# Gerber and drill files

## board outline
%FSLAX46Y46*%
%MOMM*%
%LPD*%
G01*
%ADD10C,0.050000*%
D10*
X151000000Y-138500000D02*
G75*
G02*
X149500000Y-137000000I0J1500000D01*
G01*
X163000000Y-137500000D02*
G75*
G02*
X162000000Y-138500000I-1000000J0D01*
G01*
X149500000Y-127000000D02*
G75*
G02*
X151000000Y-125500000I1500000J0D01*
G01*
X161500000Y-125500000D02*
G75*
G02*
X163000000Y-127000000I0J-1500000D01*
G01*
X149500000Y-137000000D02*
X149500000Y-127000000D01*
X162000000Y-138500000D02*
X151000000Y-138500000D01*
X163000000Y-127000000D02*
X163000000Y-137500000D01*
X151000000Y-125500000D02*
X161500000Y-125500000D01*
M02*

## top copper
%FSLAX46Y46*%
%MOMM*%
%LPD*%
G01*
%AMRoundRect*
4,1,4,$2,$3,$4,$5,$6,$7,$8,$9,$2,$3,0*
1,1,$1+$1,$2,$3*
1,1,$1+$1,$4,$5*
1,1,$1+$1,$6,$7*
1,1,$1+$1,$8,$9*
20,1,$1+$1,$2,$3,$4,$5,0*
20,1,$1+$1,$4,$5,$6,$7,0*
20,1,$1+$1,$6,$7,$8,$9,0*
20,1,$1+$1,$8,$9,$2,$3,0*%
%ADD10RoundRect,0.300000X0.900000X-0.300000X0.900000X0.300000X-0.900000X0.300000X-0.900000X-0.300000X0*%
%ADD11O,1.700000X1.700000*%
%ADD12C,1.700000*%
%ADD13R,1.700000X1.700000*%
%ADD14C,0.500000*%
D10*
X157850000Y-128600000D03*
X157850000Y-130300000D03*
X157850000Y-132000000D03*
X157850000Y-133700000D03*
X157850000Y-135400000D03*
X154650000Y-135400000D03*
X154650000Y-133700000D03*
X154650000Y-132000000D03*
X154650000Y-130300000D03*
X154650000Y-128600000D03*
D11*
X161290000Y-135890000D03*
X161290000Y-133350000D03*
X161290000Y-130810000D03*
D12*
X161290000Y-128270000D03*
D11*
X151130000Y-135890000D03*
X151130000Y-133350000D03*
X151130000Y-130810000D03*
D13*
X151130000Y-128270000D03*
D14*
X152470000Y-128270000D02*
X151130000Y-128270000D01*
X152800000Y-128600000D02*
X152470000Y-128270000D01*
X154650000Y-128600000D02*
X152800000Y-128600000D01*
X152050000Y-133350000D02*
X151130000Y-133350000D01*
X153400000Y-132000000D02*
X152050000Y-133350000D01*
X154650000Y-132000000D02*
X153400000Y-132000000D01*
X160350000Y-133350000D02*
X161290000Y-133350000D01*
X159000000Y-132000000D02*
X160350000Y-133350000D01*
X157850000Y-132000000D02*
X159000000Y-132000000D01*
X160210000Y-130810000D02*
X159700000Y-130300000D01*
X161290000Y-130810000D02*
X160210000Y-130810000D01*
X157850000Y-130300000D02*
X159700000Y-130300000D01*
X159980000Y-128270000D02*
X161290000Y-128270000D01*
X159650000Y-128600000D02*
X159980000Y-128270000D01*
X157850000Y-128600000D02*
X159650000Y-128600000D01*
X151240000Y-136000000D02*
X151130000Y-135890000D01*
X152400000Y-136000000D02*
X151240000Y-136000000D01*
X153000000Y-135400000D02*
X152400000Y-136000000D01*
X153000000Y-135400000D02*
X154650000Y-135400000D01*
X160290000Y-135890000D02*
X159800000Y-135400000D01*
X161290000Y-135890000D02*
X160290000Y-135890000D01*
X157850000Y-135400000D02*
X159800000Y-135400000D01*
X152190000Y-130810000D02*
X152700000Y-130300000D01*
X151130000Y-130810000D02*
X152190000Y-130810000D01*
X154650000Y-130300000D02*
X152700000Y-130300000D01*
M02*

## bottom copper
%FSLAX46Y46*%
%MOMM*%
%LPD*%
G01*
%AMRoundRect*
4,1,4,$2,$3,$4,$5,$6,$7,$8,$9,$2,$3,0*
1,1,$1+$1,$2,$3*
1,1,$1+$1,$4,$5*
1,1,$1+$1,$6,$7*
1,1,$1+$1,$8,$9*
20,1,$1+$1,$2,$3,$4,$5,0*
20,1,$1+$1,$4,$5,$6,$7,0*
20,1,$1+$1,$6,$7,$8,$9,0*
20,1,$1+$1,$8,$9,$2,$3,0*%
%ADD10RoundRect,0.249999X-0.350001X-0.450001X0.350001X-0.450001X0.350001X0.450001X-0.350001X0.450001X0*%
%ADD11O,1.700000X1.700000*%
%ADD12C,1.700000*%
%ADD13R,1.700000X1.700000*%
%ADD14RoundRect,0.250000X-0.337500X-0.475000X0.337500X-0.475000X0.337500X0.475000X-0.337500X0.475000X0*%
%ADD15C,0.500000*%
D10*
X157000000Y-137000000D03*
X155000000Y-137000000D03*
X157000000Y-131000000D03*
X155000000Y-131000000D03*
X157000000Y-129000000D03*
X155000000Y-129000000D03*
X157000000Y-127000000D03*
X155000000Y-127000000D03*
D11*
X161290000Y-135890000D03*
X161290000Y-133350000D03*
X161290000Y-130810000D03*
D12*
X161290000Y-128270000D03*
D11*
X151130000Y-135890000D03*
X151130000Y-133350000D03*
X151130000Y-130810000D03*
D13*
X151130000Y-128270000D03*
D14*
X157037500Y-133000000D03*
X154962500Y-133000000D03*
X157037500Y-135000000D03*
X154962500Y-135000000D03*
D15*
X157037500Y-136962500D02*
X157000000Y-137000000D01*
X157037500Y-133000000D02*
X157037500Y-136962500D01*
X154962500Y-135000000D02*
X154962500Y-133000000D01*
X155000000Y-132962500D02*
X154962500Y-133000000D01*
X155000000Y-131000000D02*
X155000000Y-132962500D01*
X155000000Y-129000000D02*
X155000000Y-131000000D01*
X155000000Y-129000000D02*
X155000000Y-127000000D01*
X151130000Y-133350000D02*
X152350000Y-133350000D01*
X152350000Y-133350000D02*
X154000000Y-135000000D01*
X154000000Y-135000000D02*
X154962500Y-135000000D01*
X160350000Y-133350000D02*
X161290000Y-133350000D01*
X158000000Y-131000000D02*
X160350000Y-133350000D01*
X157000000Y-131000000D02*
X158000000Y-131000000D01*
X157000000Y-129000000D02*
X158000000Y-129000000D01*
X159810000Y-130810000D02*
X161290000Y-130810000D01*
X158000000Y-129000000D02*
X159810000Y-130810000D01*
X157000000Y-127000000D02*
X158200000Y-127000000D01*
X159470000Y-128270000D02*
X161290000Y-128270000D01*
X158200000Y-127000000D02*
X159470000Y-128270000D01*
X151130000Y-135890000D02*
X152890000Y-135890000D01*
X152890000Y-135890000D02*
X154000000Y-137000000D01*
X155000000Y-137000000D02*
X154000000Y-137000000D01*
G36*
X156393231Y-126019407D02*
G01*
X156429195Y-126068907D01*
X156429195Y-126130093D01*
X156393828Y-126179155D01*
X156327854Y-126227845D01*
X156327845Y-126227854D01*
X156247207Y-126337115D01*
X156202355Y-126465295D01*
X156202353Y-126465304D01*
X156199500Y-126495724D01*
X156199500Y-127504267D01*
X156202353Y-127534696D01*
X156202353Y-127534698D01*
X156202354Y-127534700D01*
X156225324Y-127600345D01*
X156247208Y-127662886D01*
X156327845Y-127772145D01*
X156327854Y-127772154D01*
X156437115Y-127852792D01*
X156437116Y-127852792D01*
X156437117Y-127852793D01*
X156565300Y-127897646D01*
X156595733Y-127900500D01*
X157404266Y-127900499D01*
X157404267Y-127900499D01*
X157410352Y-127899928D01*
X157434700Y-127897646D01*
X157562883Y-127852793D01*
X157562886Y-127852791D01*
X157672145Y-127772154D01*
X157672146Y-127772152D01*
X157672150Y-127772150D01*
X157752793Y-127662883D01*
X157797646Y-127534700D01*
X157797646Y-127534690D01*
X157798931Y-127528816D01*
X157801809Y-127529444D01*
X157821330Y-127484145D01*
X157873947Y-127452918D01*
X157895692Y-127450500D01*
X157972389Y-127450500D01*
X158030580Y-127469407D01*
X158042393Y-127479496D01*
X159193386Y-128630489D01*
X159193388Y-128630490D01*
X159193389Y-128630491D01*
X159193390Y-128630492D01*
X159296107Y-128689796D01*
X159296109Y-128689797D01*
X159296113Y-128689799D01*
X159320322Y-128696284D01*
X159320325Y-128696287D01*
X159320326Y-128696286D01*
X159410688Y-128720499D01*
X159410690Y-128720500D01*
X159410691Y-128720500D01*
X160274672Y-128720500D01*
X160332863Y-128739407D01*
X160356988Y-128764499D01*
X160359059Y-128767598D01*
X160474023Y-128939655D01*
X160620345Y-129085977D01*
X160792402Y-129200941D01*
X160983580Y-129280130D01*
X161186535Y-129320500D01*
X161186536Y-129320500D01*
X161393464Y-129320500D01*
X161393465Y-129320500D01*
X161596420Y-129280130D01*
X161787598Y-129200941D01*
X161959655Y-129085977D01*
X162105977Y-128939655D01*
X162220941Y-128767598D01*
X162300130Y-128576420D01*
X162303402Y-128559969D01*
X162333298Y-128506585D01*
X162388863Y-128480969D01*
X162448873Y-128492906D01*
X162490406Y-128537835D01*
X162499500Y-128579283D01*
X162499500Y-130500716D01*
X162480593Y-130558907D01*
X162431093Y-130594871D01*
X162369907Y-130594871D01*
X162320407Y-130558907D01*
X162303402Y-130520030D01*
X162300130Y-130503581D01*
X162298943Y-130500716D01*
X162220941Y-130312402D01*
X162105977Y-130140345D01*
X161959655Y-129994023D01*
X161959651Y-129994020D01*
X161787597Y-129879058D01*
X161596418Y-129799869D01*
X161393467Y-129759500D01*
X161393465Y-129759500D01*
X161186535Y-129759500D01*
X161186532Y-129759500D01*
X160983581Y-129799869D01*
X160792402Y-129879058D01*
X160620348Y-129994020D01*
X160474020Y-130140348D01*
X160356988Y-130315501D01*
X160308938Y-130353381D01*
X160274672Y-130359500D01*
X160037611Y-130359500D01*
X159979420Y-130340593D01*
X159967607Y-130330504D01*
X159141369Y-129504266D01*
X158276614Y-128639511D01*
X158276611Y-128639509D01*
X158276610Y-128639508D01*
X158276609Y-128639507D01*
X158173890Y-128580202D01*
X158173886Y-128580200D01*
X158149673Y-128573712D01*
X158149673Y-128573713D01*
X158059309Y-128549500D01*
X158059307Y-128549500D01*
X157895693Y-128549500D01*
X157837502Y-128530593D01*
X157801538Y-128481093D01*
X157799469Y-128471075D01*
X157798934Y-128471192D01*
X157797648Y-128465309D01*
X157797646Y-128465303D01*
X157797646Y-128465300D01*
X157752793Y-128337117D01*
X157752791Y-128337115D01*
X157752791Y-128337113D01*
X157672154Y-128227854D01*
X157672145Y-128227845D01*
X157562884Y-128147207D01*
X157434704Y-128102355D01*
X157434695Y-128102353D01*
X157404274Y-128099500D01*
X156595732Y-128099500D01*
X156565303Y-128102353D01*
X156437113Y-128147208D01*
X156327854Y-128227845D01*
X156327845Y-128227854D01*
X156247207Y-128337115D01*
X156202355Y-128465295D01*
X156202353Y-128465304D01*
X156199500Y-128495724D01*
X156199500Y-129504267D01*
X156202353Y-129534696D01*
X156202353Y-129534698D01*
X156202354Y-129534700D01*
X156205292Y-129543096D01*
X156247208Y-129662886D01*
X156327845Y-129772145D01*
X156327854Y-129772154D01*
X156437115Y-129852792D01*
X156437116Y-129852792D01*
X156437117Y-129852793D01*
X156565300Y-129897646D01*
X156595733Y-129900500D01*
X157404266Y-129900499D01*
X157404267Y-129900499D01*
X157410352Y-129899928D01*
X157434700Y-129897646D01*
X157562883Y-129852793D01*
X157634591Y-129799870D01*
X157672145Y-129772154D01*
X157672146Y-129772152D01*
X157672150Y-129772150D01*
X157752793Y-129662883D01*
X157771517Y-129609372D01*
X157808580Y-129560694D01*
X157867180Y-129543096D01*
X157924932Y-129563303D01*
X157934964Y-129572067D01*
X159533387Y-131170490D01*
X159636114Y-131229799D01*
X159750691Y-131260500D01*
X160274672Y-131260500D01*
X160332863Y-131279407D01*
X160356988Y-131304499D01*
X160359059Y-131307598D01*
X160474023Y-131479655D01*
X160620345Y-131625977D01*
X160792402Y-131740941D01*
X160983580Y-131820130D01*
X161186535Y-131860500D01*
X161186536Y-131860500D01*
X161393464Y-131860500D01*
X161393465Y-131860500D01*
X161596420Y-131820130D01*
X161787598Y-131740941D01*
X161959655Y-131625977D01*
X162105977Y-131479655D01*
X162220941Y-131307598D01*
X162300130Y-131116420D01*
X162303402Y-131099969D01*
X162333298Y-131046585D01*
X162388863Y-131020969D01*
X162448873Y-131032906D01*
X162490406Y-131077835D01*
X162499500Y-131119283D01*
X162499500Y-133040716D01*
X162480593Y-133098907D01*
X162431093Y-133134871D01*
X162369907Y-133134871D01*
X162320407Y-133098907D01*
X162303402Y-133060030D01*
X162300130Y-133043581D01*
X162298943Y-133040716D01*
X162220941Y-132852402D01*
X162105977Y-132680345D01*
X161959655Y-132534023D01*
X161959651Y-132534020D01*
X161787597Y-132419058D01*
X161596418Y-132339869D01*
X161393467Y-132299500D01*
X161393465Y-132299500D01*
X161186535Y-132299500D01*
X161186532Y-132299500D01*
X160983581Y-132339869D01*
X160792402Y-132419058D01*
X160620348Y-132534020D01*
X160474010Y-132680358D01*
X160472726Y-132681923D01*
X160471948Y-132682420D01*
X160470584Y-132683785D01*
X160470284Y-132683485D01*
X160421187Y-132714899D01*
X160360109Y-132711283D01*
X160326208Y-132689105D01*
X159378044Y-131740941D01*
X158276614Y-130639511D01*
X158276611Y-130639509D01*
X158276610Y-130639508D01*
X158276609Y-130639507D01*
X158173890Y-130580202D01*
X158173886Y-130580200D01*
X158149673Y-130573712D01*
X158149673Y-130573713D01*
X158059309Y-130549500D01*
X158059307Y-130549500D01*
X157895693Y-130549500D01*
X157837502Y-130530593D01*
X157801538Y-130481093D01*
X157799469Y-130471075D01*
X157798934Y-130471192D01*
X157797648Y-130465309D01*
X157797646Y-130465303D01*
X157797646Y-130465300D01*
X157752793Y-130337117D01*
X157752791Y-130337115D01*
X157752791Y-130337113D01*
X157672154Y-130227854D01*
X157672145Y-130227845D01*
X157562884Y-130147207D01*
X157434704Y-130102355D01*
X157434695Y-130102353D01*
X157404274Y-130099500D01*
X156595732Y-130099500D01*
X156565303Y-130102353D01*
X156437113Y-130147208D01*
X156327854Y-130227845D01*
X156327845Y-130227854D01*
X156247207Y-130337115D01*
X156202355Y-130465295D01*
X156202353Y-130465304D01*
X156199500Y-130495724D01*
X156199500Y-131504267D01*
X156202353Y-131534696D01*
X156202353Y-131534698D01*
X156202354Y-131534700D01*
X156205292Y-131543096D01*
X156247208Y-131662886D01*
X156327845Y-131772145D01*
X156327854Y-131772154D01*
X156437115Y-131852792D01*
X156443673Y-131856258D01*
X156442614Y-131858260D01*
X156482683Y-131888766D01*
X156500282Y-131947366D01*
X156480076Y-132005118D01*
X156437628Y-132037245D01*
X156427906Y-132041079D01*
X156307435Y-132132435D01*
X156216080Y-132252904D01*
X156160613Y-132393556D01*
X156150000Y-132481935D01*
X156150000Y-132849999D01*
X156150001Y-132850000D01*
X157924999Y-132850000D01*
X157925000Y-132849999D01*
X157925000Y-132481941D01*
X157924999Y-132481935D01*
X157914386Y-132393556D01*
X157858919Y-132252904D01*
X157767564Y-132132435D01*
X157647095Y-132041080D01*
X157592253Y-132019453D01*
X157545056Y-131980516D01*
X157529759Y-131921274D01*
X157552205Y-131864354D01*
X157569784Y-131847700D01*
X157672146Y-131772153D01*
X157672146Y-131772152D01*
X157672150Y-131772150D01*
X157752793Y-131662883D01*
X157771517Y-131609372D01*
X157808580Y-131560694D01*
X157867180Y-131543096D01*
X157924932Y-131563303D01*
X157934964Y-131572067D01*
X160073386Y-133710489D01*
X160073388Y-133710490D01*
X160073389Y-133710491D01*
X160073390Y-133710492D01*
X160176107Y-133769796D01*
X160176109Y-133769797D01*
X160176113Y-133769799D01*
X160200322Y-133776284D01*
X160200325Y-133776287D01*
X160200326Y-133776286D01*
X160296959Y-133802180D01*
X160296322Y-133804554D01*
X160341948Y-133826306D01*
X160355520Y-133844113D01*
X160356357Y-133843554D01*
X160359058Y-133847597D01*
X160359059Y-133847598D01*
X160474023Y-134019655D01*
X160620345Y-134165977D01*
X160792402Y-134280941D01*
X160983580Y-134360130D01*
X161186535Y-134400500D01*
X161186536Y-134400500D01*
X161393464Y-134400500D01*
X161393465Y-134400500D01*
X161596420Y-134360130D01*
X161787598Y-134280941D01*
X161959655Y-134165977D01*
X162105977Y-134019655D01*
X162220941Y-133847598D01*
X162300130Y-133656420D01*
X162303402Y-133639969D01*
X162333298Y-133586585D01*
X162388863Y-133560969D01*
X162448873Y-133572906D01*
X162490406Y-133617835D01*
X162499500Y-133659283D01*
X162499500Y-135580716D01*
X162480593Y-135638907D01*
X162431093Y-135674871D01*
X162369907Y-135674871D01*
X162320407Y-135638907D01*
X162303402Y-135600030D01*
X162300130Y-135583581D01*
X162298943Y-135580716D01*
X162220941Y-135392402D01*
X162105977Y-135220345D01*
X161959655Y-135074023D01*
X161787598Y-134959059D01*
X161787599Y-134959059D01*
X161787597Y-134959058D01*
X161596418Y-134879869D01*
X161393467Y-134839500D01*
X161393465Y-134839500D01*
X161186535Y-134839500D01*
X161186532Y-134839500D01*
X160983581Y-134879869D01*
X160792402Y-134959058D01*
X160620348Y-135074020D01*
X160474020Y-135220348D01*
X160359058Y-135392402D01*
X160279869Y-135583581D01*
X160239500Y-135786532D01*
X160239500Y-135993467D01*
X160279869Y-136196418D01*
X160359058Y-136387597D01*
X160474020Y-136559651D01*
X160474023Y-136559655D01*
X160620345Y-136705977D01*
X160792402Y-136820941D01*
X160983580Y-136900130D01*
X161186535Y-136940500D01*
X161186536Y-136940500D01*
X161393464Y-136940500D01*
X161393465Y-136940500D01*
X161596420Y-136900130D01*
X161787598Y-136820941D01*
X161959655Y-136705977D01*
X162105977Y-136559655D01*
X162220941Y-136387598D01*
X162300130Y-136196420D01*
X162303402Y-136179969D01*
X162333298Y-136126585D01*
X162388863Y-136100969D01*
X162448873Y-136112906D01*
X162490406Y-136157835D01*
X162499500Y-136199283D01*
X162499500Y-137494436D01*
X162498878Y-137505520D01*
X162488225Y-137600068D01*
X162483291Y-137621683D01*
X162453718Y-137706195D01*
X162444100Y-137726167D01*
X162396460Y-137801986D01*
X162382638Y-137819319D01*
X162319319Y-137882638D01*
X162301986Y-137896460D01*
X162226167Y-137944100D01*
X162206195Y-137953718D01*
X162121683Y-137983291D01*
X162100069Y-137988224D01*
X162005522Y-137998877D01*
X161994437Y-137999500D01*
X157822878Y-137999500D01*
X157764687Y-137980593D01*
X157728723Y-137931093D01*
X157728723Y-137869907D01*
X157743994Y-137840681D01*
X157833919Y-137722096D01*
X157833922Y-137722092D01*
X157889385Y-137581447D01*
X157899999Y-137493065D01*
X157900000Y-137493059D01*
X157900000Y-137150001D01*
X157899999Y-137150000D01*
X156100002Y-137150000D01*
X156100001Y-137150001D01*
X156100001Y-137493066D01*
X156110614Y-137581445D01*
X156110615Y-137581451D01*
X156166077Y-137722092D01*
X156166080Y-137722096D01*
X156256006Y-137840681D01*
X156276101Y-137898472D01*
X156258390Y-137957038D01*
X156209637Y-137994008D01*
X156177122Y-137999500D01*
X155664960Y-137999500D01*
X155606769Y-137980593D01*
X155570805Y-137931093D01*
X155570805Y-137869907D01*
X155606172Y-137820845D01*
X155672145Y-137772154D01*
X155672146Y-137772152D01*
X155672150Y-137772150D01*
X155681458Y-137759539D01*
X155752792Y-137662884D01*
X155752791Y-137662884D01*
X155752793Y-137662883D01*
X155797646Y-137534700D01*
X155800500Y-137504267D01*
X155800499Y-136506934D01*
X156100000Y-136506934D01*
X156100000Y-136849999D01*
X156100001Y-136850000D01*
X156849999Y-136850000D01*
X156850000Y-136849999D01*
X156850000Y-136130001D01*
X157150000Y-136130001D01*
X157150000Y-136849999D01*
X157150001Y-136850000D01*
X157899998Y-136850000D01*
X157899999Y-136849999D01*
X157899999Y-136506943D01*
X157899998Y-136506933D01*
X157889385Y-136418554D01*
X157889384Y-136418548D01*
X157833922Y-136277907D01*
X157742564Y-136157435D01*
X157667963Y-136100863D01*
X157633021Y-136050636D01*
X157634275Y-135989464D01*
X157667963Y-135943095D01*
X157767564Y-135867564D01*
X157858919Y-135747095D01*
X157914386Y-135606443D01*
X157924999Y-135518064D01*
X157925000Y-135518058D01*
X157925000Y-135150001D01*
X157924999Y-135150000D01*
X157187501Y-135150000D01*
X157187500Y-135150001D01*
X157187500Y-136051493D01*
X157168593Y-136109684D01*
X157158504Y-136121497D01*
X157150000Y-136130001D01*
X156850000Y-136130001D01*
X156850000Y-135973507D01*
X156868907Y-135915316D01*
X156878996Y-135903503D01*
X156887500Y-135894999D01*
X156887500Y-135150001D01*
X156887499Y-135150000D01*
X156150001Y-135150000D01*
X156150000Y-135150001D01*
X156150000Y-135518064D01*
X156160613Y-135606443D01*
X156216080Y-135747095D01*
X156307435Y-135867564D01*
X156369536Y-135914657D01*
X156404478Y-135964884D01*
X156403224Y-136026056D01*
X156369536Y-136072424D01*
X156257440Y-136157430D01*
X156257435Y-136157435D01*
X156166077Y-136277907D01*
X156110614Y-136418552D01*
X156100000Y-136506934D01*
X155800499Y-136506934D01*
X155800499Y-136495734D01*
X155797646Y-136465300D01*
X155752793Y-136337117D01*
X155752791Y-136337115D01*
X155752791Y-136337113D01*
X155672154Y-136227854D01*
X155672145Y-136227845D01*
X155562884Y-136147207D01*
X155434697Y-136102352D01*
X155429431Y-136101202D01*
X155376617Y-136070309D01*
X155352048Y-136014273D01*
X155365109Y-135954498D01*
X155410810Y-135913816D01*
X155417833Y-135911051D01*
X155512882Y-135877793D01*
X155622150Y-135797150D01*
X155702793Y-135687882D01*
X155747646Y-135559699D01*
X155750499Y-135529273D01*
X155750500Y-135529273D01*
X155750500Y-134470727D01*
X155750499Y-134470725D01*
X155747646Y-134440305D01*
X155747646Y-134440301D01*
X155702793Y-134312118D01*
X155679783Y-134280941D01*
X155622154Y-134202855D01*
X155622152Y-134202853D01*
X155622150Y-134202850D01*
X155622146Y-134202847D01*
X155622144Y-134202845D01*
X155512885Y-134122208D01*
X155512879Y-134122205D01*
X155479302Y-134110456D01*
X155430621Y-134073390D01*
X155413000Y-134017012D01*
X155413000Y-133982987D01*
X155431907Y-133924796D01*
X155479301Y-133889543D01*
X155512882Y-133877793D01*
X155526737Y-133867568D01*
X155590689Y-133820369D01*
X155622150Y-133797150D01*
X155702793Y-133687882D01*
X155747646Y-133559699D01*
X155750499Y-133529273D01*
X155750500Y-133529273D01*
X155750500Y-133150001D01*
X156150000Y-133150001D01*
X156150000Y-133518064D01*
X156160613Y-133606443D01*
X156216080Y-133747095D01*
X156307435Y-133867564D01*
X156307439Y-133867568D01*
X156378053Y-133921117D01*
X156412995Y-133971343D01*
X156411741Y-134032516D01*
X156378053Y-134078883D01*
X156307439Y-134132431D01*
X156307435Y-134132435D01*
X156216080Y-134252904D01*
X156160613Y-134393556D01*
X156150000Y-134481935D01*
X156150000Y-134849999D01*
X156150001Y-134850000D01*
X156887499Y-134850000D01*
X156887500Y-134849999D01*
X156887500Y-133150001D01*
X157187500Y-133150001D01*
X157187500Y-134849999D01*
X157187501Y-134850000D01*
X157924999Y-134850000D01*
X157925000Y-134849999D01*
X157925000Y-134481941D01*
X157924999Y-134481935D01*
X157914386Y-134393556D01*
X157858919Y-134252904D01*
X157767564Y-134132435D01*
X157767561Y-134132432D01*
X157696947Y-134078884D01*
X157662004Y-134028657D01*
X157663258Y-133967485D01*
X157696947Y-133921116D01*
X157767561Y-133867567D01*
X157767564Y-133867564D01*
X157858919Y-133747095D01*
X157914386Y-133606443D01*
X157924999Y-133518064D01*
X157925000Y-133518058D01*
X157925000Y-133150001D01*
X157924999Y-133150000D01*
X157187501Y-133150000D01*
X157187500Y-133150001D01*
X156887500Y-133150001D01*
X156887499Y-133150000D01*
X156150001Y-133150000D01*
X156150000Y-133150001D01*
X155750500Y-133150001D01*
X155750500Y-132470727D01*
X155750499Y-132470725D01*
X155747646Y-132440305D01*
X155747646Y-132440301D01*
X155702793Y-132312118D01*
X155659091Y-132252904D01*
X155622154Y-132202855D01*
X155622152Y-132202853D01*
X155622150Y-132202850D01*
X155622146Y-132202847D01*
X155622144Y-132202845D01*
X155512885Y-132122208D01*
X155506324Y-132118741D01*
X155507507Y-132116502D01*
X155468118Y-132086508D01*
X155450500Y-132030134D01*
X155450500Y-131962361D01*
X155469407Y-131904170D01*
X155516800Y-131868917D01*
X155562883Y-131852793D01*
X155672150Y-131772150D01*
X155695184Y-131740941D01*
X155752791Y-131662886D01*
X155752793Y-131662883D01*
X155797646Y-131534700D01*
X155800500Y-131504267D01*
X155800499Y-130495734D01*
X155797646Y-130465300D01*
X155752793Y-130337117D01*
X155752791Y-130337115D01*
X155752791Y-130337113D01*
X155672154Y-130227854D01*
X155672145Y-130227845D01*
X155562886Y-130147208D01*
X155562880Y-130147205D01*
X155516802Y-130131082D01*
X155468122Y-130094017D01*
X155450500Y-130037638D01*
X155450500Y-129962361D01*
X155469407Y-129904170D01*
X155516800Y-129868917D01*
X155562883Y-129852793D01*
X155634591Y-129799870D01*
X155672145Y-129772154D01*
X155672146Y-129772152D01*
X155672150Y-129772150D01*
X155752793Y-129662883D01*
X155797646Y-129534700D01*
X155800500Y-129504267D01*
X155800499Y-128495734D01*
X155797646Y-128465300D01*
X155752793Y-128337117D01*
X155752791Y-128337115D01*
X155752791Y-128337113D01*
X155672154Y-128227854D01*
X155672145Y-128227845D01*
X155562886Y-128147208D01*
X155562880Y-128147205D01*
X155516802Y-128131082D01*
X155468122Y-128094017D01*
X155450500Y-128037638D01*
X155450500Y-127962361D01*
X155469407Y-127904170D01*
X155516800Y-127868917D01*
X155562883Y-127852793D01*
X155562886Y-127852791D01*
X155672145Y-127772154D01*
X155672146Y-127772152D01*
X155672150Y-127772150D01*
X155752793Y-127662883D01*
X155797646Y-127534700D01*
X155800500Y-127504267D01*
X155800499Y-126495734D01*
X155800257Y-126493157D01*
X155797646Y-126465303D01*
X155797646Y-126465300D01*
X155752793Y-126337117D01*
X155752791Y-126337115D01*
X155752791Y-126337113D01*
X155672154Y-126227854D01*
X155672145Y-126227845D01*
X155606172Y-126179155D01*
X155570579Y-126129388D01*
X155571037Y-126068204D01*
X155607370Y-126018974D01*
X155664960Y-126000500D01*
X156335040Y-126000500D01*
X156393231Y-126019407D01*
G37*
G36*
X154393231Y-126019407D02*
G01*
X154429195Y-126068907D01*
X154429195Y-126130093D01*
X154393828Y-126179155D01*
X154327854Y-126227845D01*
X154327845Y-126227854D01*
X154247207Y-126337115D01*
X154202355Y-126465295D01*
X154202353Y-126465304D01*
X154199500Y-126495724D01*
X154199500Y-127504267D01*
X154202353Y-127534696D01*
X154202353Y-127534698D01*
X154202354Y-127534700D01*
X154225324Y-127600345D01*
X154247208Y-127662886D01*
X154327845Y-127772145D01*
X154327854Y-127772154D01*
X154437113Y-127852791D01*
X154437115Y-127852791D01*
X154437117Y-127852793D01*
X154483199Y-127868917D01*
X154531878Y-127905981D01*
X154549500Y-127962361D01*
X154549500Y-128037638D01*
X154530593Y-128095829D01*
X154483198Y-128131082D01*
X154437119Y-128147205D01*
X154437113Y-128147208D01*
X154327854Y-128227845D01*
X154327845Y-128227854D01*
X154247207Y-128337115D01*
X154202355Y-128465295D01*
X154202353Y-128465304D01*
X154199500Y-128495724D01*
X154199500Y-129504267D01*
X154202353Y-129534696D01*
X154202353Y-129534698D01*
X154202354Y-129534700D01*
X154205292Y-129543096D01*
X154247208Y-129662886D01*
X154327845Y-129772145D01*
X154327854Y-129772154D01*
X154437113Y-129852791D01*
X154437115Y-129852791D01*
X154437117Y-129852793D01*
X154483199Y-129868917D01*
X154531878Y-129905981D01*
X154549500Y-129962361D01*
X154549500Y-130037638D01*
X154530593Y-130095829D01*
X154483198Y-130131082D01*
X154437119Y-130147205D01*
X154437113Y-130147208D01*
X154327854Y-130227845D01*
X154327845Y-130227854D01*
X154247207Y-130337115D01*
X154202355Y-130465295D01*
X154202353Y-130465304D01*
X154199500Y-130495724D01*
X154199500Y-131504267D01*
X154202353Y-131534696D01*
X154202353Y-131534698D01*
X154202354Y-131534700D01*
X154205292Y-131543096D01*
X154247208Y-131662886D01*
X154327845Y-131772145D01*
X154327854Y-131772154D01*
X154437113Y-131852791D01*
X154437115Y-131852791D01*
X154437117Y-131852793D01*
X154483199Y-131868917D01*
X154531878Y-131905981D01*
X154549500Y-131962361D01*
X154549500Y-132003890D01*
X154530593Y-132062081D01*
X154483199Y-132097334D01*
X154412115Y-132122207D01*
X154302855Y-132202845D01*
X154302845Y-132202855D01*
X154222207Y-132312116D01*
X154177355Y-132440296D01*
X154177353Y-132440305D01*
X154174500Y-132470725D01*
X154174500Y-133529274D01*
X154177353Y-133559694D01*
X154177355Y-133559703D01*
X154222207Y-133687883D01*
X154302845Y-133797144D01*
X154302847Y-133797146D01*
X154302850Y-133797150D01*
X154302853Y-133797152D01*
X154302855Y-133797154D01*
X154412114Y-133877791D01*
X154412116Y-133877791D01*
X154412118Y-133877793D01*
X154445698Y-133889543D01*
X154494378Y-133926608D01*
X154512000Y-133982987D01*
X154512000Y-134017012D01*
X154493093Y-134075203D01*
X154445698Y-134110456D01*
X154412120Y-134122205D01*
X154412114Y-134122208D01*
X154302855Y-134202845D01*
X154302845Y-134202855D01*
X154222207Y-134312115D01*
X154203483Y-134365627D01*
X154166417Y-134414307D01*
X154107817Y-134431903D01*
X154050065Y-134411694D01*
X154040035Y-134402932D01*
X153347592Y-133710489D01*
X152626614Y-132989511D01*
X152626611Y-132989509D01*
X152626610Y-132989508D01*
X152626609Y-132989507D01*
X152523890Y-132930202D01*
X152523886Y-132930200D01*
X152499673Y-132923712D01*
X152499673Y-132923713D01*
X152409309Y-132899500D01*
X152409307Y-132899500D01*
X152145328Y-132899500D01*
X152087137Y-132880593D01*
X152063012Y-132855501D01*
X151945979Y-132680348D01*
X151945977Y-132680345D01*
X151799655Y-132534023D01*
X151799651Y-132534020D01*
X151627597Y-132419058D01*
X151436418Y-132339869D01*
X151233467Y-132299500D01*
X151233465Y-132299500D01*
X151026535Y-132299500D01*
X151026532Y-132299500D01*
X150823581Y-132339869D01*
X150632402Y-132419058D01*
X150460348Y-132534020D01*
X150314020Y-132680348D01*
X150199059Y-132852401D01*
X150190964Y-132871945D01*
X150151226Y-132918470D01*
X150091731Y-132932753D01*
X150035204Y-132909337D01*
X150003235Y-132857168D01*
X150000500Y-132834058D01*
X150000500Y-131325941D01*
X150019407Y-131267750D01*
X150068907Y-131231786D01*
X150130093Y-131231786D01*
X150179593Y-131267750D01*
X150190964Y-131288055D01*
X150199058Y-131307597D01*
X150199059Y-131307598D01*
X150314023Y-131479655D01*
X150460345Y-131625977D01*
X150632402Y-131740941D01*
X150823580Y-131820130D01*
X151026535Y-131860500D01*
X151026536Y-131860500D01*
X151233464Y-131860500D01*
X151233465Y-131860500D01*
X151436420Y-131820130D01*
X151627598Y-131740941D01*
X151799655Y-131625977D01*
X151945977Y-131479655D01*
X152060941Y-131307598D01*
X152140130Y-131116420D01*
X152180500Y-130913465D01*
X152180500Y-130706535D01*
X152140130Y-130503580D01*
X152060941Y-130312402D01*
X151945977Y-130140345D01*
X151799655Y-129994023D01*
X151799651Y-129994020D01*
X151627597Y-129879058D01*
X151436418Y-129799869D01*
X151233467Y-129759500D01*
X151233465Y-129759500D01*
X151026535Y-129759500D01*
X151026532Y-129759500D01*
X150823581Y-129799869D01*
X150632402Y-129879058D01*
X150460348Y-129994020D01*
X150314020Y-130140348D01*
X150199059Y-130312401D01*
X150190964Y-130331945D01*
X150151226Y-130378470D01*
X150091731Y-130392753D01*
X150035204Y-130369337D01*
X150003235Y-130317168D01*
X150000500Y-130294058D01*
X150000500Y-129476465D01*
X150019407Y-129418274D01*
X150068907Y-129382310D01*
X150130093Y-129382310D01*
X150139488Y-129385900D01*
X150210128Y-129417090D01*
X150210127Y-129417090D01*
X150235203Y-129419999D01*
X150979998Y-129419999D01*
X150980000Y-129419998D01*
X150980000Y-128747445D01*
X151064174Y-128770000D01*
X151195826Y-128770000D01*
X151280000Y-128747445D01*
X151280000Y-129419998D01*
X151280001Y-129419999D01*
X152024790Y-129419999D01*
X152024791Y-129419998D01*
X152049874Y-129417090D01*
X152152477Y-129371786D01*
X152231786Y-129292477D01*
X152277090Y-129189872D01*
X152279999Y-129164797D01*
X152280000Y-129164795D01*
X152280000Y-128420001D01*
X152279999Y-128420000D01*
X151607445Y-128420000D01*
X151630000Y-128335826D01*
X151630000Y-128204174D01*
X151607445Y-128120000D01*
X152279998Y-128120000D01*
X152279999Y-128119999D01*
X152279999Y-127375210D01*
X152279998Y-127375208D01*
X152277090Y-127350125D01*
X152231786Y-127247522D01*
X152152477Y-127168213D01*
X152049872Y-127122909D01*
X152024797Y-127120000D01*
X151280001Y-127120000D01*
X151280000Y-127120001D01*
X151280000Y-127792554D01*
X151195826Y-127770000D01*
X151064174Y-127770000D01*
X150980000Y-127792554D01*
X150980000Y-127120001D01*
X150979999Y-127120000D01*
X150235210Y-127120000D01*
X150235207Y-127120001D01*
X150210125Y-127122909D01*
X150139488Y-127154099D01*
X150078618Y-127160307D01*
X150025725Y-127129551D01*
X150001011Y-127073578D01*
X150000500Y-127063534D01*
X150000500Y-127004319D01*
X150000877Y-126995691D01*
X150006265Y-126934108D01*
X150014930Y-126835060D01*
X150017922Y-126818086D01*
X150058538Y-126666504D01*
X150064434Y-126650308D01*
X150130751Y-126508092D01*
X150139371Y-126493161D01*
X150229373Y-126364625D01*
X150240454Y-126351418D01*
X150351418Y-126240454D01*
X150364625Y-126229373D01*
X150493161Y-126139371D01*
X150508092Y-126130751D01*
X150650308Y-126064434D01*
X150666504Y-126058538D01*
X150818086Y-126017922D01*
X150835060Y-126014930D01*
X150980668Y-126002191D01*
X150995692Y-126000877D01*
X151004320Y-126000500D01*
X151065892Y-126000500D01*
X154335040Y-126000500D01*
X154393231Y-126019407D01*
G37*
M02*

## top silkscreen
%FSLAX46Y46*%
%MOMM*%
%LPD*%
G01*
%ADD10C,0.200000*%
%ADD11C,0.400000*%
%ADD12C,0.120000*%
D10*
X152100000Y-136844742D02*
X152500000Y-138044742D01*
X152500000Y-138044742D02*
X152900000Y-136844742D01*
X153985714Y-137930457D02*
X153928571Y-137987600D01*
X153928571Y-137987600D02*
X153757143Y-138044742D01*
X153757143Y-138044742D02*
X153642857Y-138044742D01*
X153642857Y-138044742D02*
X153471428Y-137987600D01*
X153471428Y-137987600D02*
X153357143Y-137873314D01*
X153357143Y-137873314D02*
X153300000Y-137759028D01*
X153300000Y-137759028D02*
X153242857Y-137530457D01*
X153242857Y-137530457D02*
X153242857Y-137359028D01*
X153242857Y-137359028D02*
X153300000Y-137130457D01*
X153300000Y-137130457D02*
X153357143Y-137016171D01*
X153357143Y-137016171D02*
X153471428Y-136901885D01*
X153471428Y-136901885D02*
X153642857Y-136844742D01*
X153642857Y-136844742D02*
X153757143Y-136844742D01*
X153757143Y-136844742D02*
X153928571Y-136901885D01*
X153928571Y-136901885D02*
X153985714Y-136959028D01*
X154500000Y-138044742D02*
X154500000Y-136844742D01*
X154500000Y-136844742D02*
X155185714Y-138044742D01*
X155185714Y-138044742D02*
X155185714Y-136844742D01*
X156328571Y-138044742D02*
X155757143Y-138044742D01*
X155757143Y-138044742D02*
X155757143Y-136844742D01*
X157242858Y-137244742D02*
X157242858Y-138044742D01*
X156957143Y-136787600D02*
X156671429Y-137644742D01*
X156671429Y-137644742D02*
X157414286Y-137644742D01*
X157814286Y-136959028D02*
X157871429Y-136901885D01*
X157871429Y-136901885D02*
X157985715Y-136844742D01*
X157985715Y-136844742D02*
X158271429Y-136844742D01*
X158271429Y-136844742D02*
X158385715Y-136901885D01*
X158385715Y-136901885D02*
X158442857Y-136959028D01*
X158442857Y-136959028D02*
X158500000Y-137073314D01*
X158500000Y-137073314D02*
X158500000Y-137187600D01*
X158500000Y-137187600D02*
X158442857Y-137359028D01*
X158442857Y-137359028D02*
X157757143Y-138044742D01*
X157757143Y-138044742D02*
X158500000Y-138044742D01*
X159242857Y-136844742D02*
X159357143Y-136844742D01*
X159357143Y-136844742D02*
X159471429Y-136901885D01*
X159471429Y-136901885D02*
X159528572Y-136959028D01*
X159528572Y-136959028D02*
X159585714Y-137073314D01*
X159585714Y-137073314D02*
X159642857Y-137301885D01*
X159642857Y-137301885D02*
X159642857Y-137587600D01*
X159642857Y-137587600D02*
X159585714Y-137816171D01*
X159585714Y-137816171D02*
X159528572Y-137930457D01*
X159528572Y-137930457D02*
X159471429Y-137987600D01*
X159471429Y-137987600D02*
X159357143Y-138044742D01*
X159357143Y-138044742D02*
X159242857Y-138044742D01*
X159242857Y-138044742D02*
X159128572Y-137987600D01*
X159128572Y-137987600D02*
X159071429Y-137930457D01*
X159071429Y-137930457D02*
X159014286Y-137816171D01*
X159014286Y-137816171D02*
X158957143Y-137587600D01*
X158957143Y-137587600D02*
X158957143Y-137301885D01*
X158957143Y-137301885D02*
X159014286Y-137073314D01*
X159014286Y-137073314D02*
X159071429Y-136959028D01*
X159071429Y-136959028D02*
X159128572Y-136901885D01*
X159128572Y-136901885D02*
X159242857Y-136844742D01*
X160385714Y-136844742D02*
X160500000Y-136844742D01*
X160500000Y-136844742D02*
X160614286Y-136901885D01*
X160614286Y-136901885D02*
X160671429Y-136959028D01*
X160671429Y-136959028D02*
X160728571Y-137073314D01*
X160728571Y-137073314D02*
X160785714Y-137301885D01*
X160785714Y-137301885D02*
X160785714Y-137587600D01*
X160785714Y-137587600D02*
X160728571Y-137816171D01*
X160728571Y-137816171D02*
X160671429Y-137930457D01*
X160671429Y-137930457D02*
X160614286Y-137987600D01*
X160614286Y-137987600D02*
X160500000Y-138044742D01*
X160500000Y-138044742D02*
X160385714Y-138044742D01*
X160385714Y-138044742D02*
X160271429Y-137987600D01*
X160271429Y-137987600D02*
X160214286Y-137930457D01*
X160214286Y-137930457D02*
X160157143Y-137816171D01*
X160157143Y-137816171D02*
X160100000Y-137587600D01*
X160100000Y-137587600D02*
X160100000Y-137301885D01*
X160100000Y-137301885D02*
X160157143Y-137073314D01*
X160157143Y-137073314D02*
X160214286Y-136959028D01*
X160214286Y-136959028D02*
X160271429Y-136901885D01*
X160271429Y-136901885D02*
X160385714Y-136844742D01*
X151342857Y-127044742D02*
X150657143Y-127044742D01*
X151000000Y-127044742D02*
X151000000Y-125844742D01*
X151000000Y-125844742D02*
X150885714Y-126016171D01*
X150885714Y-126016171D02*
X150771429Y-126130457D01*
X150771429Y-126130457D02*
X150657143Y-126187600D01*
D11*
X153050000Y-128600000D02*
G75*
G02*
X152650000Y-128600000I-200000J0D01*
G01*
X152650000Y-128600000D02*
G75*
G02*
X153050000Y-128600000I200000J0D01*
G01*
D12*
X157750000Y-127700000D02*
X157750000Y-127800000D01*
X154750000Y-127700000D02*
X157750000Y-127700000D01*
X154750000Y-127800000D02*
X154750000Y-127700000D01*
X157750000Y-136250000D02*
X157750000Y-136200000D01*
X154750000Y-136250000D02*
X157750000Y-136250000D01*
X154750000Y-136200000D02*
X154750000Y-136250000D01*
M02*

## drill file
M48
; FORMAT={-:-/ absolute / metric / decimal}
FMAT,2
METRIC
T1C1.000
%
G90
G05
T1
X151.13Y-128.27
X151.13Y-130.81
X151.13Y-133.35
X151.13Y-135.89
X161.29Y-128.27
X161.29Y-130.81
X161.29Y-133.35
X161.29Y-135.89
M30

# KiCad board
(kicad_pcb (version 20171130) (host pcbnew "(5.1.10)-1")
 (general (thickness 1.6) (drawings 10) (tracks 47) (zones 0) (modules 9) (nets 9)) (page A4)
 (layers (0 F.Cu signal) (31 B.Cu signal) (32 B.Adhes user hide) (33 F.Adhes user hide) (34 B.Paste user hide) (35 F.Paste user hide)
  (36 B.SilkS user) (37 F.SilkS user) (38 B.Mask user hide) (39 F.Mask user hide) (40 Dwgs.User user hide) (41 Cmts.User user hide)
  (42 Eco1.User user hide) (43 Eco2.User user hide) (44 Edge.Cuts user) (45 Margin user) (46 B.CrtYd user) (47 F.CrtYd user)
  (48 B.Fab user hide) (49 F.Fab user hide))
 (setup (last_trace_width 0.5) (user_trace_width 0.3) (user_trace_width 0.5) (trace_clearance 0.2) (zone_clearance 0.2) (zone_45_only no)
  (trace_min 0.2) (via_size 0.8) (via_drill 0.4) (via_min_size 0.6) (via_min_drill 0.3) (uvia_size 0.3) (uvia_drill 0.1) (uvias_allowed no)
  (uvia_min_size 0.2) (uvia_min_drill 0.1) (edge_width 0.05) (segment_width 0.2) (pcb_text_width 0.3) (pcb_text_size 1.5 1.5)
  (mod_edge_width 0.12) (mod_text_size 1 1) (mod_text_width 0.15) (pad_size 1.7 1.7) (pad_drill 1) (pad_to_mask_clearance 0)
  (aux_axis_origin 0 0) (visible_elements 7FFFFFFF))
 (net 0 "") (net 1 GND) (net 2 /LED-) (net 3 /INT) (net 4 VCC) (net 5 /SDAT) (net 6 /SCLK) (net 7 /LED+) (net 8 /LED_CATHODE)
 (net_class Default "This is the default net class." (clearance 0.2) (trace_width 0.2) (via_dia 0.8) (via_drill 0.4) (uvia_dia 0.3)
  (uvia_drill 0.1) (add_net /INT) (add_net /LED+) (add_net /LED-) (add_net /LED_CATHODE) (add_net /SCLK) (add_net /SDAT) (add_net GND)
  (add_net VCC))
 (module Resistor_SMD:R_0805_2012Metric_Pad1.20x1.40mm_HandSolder (layer B.Cu) (at 156 137)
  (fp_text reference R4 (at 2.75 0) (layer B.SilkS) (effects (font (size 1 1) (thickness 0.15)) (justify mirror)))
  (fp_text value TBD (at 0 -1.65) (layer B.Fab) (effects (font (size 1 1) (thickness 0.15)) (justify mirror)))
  (pad 2 smd roundrect (at 1 0) (size 1.2 1.4) (layers B.Cu B.Paste B.Mask) (roundrect_rratio 0.2083325) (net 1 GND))
  (pad 1 smd roundrect (at -1 0) (size 1.2 1.4) (layers B.Cu B.Paste B.Mask) (roundrect_rratio 0.2083325) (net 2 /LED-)))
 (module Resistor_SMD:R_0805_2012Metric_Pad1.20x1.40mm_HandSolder (layer B.Cu) (at 156 131)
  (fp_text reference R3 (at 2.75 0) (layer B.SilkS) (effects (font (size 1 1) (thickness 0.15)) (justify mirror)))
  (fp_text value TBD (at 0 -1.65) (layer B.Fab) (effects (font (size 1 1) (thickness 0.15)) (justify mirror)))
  (pad 2 smd roundrect (at 1 0) (size 1.2 1.4) (layers B.Cu B.Paste B.Mask) (roundrect_rratio 0.2083325) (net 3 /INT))
  (pad 1 smd roundrect (at -1 0) (size 1.2 1.4) (layers B.Cu B.Paste B.Mask) (roundrect_rratio 0.2083325) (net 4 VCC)))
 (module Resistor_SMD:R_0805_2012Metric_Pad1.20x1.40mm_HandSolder (layer B.Cu) (at 156 129)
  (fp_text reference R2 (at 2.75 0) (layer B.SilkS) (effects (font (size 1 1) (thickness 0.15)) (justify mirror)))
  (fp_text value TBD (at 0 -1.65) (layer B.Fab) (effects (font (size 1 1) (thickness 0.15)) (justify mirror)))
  (pad 2 smd roundrect (at 1 0) (size 1.2 1.4) (layers B.Cu B.Paste B.Mask) (roundrect_rratio 0.2083325) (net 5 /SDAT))
  (pad 1 smd roundrect (at -1 0) (size 1.2 1.4) (layers B.Cu B.Paste B.Mask) (roundrect_rratio 0.2083325) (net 4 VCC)))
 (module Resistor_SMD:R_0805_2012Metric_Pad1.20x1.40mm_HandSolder (layer B.Cu) (at 156 127)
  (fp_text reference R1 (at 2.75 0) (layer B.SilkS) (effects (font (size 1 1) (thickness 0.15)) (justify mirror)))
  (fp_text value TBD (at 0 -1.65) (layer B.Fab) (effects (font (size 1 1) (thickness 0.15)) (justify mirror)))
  (pad 2 smd roundrect (at 1 0) (size 1.2 1.4) (layers B.Cu B.Paste B.Mask) (roundrect_rratio 0.2083325) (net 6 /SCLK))
  (pad 1 smd roundrect (at -1 0) (size 1.2 1.4) (layers B.Cu B.Paste B.Mask) (roundrect_rratio 0.2083325) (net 4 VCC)))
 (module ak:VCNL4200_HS (layer F.Cu) (at 156.25 132 90)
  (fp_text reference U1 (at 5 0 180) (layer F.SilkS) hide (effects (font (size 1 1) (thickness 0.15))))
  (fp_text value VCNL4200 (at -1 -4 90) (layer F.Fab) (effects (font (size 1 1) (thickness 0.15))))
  (fp_circle (center 3.4 -3.4) (end 3.6 -3.4) (layer F.SilkS) (width 0.4))
  (fp_line (start 4.3 1.5) (end 4.2 1.5) (layer F.SilkS) (width 0.12))
  (fp_line (start 4.3 -1.5) (end 4.3 1.5) (layer F.SilkS) (width 0.12))
  (fp_line (start 4.2 -1.5) (end 4.3 -1.5) (layer F.SilkS) (width 0.12))
  (fp_line (start -4.25 1.5) (end -4.2 1.5) (layer F.SilkS) (width 0.12))
  (fp_line (start -4.25 -1.5) (end -4.25 1.5) (layer F.SilkS) (width 0.12))
  (fp_line (start -4.2 -1.5) (end -4.25 -1.5) (layer F.SilkS) (width 0.12))
  (pad 10 smd roundrect (at 3.4 1.6 90) (size 1.2 2.4) (layers F.Cu F.Paste F.Mask) (roundrect_rratio 0.25) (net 6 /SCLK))
  (pad 9 smd roundrect (at 1.7 1.6 90) (size 1.2 2.4) (layers F.Cu F.Paste F.Mask) (roundrect_rratio 0.25) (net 5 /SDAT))
  (pad 8 smd roundrect (at 0 1.6 90) (size 1.2 2.4) (layers F.Cu F.Paste F.Mask) (roundrect_rratio 0.25) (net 3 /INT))
  (pad 7 smd roundrect (at -1.7 1.6 90) (size 1.2 2.4) (layers F.Cu F.Paste F.Mask) (roundrect_rratio 0.25))
  (pad 6 smd roundrect (at -3.4 1.6 90) (size 1.2 2.4) (layers F.Cu F.Paste F.Mask) (roundrect_rratio 0.25) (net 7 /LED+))
  (pad 5 smd roundrect (at -3.4 -1.6 90) (size 1.2 2.4) (layers F.Cu F.Paste F.Mask) (roundrect_rratio 0.25) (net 2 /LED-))
  (pad 4 smd roundrect (at -1.7 -1.6 90) (size 1.2 2.4) (layers F.Cu F.Paste F.Mask) (roundrect_rratio 0.25))
  (pad 3 smd roundrect (at 0 -1.6 90) (size 1.2 2.4) (layers F.Cu F.Paste F.Mask) (roundrect_rratio 0.25) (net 4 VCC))
  (pad 2 smd roundrect (at 1.7 -1.6 90) (size 1.2 2.4) (layers F.Cu F.Paste F.Mask) (roundrect_rratio 0.25) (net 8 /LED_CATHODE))
  (pad 1 smd roundrect (at 3.4 -1.6 90) (size 1.2 2.4) (layers F.Cu F.Paste F.Mask) (roundrect_rratio 0.25) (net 1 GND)))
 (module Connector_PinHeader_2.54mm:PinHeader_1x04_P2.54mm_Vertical (layer B.Cu) (at 161.29 128.27 180)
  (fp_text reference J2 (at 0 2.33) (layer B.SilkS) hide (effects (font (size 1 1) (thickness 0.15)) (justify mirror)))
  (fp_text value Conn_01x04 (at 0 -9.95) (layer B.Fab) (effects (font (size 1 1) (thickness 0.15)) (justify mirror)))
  (pad 4 thru_hole oval (at 0 -7.62 180) (size 1.7 1.7) (drill 1) (layers *.Cu *.Mask) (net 7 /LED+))
  (pad 3 thru_hole oval (at 0 -5.08 180) (size 1.7 1.7) (drill 1) (layers *.Cu *.Mask) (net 3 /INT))
  (pad 2 thru_hole oval (at 0 -2.54 180) (size 1.7 1.7) (drill 1) (layers *.Cu *.Mask) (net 5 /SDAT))
  (pad 1 thru_hole circle (at 0 0 180) (size 1.7 1.7) (drill 1) (layers *.Cu *.Mask) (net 6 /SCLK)))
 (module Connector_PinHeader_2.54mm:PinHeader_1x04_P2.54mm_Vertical (layer B.Cu) (at 151.13 128.27 180)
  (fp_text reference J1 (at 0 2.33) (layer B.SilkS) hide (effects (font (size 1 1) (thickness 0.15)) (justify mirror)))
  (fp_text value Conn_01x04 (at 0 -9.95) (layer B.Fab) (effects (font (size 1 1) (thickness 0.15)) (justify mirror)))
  (pad 4 thru_hole oval (at 0 -7.62 180) (size 1.7 1.7) (drill 1) (layers *.Cu *.Mask) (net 2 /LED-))
  (pad 3 thru_hole oval (at 0 -5.08 180) (size 1.7 1.7) (drill 1) (layers *.Cu *.Mask) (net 4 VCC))
  (pad 2 thru_hole oval (at 0 -2.54 180) (size 1.7 1.7) (drill 1) (layers *.Cu *.Mask) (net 8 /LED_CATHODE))
  (pad 1 thru_hole rect (at 0 0 180) (size 1.7 1.7) (drill 1) (layers *.Cu *.Mask) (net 1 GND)))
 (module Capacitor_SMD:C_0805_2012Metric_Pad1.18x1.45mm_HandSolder (layer B.Cu) (at 156 133)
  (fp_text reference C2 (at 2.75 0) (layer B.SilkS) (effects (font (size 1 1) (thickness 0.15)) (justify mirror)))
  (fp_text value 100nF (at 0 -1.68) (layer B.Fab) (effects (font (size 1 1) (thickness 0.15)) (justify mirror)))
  (pad 2 smd roundrect (at 1.0375 0) (size 1.175 1.45) (layers B.Cu B.Paste B.Mask) (roundrect_rratio 0.2127659574468085) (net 1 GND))
  (pad 1 smd roundrect (at -1.0375 0) (size 1.175 1.45) (layers B.Cu B.Paste B.Mask) (roundrect_rratio 0.2127659574468085) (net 4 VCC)))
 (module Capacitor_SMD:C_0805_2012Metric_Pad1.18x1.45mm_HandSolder (layer B.Cu) (at 156 135)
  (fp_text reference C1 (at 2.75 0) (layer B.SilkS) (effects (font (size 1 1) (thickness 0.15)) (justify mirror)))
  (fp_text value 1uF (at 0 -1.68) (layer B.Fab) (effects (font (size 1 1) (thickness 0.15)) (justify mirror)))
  (pad 2 smd roundrect (at 1.0375 0) (size 1.175 1.45) (layers B.Cu B.Paste B.Mask) (roundrect_rratio 0.2127659574468085) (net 1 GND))
  (pad 1 smd roundrect (at -1.0375 0) (size 1.175 1.45) (layers B.Cu B.Paste B.Mask) (roundrect_rratio 0.2127659574468085) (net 4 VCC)))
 (gr_arc (start 151 137) (end 149.5 137) (angle -90) (layer Edge.Cuts) (width 0.05))
 (gr_arc (start 162 137.5) (end 162 138.5) (angle -90) (layer Edge.Cuts) (width 0.05))
 (gr_arc (start 151 127) (end 151 125.5) (angle -90) (layer Edge.Cuts) (width 0.05))
 (gr_arc (start 161.5 127) (end 163 127) (angle -90) (layer Edge.Cuts) (width 0.05))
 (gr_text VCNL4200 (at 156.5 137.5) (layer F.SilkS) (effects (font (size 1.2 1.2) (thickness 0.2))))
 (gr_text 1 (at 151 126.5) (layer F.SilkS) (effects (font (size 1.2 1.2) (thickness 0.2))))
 (gr_line (start 149.5 137) (end 149.5 127) (layer Edge.Cuts) (width 0.05))
 (gr_line (start 162 138.5) (end 151 138.5) (layer Edge.Cuts) (width 0.05))
 (gr_line (start 163 127) (end 163 137.5) (layer Edge.Cuts) (width 0.05))
 (gr_line (start 151 125.5) (end 161.5 125.5) (layer Edge.Cuts) (width 0.05))
 (segment (start 157.0375 136.9625) (end 157 137) (width 0.5) (layer B.Cu) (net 1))
 (segment (start 157.0375 133) (end 157.0375 136.9625) (width 0.5) (layer B.Cu) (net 1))
 (segment (start 152.47 128.27) (end 151.13 128.27) (width 0.5) (layer F.Cu) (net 1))
 (segment (start 152.8 128.6) (end 152.47 128.27) (width 0.5) (layer F.Cu) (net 1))
 (segment (start 154.65 128.6) (end 152.8 128.6) (width 0.5) (layer F.Cu) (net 1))
 (segment (start 154.9625 135) (end 154.9625 133) (width 0.5) (layer B.Cu) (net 4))
 (segment (start 155 132.9625) (end 154.9625 133) (width 0.5) (layer B.Cu) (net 4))
 (segment (start 155 131) (end 155 132.9625) (width 0.5) (layer B.Cu) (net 4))
 (segment (start 155 129) (end 155 131) (width 0.5) (layer B.Cu) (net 4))
 (segment (start 155 129) (end 155 127) (width 0.5) (layer B.Cu) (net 4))
 (segment (start 152.05 133.35) (end 151.13 133.35) (width 0.5) (layer F.Cu) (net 4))
 (segment (start 153.4 132) (end 152.05 133.35) (width 0.5) (layer F.Cu) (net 4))
 (segment (start 154.65 132) (end 153.4 132) (width 0.5) (layer F.Cu) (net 4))
 (segment (start 151.13 133.35) (end 152.35 133.35) (width 0.5) (layer B.Cu) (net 4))
 (segment (start 152.35 133.35) (end 154 135) (width 0.5) (layer B.Cu) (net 4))
 (segment (start 154 135) (end 154.9625 135) (width 0.5) (layer B.Cu) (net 4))
 (segment (start 160.35 133.35) (end 161.29 133.35) (width 0.5) (layer B.Cu) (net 3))
 (segment (start 158 131) (end 160.35 133.35) (width 0.5) (layer B.Cu) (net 3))
 (segment (start 157 131) (end 158 131) (width 0.5) (layer B.Cu) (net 3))
 (segment (start 160.35 133.35) (end 161.29 133.35) (width 0.5) (layer F.Cu) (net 3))
 (segment (start 159 132) (end 160.35 133.35) (width 0.5) (layer F.Cu) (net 3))
 (segment (start 157.85 132) (end 159 132) (width 0.5) (layer F.Cu) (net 3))
 (segment (start 157 129) (end 158 129) (width 0.5) (layer B.Cu) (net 5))
 (segment (start 159.81 130.81) (end 161.29 130.81) (width 0.5) (layer B.Cu) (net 5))
 (segment (start 158 129) (end 159.81 130.81) (width 0.5) (layer B.Cu) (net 5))
 (segment (start 160.21 130.81) (end 159.7 130.3) (width 0.5) (layer F.Cu) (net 5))
 (segment (start 161.29 130.81) (end 160.21 130.81) (width 0.5) (layer F.Cu) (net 5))
 (segment (start 157.85 130.3) (end 159.7 130.3) (width 0.5) (layer F.Cu) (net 5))
 (segment (start 157 127) (end 158.2 127) (width 0.5) (layer B.Cu) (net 6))
 (segment (start 159.47 128.27) (end 161.29 128.27) (width 0.5) (layer B.Cu) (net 6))
 (segment (start 158.2 127) (end 159.47 128.27) (width 0.5) (layer B.Cu) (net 6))
 (segment (start 159.98 128.27) (end 161.29 128.27) (width 0.5) (layer F.Cu) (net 6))
 (segment (start 159.65 128.6) (end 159.98 128.27) (width 0.5) (layer F.Cu) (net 6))
 (segment (start 157.85 128.6) (end 159.65 128.6) (width 0.5) (layer F.Cu) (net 6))
 (segment (start 151.13 135.89) (end 152.89 135.89) (width 0.5) (layer B.Cu) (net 2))
 (segment (start 152.89 135.89) (end 154 137) (width 0.5) (layer B.Cu) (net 2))
 (segment (start 155 137) (end 154 137) (width 0.5) (layer B.Cu) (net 2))
 (segment (start 151.24 136) (end 151.13 135.89) (width 0.5) (layer F.Cu) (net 2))
 (segment (start 152.4 136) (end 151.24 136) (width 0.5) (layer F.Cu) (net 2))
 (segment (start 153 135.4) (end 152.4 136) (width 0.5) (layer F.Cu) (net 2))
 (segment (start 153 135.4) (end 154.65 135.4) (width 0.5) (layer F.Cu) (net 2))
 (segment (start 160.29 135.89) (end 159.8 135.4) (width 0.5) (layer F.Cu) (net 7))
 (segment (start 161.29 135.89) (end 160.29 135.89) (width 0.5) (layer F.Cu) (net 7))
 (segment (start 157.85 135.4) (end 159.8 135.4) (width 0.5) (layer F.Cu) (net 7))
 (segment (start 152.19 130.81) (end 152.7 130.3) (width 0.5) (layer F.Cu) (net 8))
 (segment (start 151.13 130.81) (end 152.19 130.81) (width 0.5) (layer F.Cu) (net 8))
 (segment (start 154.65 130.3) (end 152.7 130.3) (width 0.5) (layer F.Cu) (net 8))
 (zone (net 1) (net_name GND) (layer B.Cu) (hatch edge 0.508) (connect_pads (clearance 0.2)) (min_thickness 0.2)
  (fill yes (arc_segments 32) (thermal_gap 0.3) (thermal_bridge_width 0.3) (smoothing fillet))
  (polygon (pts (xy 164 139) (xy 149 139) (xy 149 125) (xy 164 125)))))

